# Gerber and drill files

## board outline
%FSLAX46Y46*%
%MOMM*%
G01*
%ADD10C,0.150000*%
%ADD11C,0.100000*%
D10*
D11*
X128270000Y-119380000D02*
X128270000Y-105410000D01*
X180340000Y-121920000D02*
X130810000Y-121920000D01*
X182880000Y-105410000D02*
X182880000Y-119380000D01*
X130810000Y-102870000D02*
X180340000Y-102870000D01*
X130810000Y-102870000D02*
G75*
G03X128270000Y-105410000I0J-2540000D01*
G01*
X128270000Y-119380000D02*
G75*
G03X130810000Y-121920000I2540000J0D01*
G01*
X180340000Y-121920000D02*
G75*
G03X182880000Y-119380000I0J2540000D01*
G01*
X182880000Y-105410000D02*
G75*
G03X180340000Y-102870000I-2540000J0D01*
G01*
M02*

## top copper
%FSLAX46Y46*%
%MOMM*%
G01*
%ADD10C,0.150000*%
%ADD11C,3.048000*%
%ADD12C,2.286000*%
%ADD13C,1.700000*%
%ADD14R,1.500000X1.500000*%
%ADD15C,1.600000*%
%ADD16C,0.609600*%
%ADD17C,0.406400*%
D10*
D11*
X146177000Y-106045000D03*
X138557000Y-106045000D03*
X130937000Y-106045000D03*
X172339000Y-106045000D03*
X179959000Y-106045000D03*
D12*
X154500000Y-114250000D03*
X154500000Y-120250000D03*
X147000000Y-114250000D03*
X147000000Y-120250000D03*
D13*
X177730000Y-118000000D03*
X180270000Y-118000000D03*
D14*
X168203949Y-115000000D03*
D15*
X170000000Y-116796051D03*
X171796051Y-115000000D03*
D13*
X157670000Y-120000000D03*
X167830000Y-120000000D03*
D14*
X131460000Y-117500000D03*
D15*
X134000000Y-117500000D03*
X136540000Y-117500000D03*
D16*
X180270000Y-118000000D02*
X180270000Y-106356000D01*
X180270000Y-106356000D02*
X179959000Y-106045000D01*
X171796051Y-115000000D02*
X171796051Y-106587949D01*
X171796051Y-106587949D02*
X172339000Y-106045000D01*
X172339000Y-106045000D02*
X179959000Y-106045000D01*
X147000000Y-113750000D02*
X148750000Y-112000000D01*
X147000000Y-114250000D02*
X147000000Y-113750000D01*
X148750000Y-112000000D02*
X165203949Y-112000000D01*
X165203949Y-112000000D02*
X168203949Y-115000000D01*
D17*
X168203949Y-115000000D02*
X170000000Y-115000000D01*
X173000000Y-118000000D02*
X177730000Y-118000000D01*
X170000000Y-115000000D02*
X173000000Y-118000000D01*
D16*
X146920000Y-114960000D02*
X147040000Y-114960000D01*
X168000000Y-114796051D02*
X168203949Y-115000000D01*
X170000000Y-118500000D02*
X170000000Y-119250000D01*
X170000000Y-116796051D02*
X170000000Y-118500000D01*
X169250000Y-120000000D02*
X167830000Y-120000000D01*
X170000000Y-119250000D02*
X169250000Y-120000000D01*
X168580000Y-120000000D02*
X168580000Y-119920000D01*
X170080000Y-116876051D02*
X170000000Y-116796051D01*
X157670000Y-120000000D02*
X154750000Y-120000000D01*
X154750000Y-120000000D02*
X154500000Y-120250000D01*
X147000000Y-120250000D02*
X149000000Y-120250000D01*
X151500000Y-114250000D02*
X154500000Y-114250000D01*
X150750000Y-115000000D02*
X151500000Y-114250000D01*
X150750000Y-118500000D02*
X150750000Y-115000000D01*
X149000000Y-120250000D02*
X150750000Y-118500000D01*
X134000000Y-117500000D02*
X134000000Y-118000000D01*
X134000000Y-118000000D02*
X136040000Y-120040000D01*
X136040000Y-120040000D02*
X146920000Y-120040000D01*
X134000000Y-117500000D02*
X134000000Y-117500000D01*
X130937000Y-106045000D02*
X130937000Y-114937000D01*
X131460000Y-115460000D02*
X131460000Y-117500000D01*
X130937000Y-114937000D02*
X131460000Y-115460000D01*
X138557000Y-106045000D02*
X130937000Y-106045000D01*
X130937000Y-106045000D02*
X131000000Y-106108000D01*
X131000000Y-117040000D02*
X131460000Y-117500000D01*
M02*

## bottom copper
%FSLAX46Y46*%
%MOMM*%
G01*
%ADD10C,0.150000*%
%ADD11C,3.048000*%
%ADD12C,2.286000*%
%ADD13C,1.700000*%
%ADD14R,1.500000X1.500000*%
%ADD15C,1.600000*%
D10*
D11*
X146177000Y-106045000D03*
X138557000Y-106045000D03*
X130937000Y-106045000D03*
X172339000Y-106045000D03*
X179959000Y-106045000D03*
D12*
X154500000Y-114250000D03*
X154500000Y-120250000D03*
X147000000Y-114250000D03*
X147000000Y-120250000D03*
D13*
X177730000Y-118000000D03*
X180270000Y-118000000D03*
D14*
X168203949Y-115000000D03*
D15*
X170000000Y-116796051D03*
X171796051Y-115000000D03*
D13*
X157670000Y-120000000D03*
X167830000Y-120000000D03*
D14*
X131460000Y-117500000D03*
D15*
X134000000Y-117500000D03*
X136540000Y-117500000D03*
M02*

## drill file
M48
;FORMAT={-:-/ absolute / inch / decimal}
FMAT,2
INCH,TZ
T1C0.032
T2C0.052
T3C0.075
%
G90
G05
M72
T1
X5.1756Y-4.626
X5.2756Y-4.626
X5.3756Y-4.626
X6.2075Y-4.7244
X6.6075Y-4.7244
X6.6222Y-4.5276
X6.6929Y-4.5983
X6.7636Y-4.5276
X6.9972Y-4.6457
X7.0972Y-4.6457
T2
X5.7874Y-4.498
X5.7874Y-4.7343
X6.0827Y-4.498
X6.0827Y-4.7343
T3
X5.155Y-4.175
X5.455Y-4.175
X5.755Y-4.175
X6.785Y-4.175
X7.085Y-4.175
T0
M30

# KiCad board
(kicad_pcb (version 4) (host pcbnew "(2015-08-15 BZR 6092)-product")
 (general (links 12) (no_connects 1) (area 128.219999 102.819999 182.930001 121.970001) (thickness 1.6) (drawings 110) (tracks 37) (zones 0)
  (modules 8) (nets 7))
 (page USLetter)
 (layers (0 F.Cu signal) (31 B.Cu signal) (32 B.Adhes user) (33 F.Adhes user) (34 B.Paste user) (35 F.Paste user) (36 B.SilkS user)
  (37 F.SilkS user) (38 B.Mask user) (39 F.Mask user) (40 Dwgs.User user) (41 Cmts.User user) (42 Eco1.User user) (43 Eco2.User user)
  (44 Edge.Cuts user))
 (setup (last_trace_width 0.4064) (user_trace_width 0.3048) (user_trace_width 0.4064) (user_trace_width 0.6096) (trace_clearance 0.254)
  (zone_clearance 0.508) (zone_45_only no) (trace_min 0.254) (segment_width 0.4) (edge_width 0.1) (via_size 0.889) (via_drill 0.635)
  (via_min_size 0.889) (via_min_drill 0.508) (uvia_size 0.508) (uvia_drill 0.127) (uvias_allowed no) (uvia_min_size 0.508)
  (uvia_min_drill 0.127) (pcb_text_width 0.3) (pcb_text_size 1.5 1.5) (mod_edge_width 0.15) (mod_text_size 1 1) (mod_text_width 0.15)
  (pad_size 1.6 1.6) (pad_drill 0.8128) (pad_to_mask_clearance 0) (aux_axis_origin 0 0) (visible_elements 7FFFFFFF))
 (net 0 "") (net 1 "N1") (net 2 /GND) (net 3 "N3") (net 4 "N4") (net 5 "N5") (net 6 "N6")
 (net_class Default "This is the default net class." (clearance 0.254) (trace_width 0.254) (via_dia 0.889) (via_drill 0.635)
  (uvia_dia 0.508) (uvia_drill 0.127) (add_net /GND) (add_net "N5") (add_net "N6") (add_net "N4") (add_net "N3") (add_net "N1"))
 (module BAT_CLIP (layer F.Cu) (at 155.575 106.045)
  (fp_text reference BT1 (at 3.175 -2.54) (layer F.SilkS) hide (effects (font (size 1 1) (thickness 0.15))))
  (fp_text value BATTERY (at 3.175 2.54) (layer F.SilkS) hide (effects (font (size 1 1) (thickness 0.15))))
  (pad 1 thru_hole circle (at -9.398 0) (size 3.048 3.048) (drill 1.905) (layers *.Cu *.Mask) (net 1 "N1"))
  (pad 1 thru_hole circle (at -17.018 0) (size 3.048 3.048) (drill 1.905) (layers *.Cu *.Mask) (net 1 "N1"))
  (pad 1 thru_hole circle (at -24.638 0) (size 3.048 3.048) (drill 1.905) (layers *.Cu *.Mask) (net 1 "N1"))
  (pad 2 thru_hole circle (at 16.764 0) (size 3.048 3.048) (drill 1.905) (layers *.Cu *.Mask) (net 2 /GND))
  (pad 2 thru_hole circle (at 24.384 0) (size 3.048 3.048) (drill 1.905) (layers *.Cu *.Mask) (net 2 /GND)))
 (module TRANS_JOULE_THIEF (layer F.Cu) (at 152 117.25 270)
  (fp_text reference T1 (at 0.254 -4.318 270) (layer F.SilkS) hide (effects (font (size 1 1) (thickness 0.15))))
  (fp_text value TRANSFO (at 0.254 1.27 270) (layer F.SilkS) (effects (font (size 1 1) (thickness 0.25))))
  (pad 1 thru_hole circle (at -3 -2.5 270) (size 2.286 2.286) (drill 1.3208) (layers *.Cu B.Mask) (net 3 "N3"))
  (pad 2 thru_hole circle (at 3 -2.5 270) (size 2.286 2.286) (drill 1.3208) (layers *.Cu B.Mask) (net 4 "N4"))
  (pad 3 thru_hole circle (at -3 5 270) (size 2.286 2.286) (drill 1.3208) (layers *.Cu B.Mask) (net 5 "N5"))
  (pad 4 thru_hole circle (at 3 5 270) (size 2.286 2.286) (drill 1.3208) (layers *.Cu B.Mask) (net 3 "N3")))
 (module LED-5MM (layer F.Cu) (at 179 118)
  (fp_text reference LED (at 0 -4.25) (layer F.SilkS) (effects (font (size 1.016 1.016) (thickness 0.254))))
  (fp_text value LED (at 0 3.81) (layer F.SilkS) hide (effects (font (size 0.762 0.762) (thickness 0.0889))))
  (pad 1 thru_hole circle (at -1.27 0) (size 1.7 1.7) (drill 0.8128) (layers *.Cu B.Mask) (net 5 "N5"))
  (pad 2 thru_hole circle (at 1.27 0) (size 1.7 1.7) (drill 0.8128) (layers *.Cu B.Mask) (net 2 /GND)))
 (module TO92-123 (layer F.Cu) (at 170 115 135)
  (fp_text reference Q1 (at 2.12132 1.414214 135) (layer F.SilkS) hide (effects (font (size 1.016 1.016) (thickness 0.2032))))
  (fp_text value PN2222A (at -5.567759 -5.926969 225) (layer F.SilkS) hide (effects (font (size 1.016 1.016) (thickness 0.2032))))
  (pad 3 thru_hole rect (at 1.27 -1.27 180) (size 1.5 1.5) (drill 0.8128) (layers *.Cu B.Mask) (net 5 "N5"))
  (pad 2 thru_hole circle (at -1.27 -1.27 135) (size 1.6 1.6) (drill 0.8128) (layers *.Cu B.Mask) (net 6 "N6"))
  (pad 1 thru_hole circle (at -1.27 1.27 135) (size 1.6 1.6) (drill 0.8128) (layers *.Cu B.Mask) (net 2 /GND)))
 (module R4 (layer F.Cu) (at 162.75 120) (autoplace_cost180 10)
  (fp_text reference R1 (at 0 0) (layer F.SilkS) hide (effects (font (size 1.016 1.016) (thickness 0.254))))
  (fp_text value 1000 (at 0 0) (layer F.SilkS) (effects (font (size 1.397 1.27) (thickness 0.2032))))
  (pad 1 thru_hole circle (at -5.08 0) (size 1.7 1.7) (drill 0.8128) (layers *.Cu B.Mask) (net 4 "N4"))
  (pad 2 thru_hole circle (at 5.08 0) (size 1.7 1.7) (drill 0.8128) (layers *.Cu B.Mask) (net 6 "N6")))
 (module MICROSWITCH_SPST (layer F.Cu) (at 134 117.5)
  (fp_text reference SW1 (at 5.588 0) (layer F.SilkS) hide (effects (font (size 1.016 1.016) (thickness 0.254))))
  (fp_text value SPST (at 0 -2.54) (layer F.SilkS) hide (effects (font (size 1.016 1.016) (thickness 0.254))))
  (pad 1 thru_hole rect (at -2.54 0) (size 1.5 1.5) (drill 0.8128) (layers *.Cu B.Mask) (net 1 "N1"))
  (pad 2 thru_hole circle (at 0 0) (size 1.6 1.6) (drill 0.8128) (layers *.Cu B.Mask) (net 3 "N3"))
  (pad 3 thru_hole circle (at 2.54 0) (size 1.6 1.6) (drill 0.8128) (layers *.Cu B.Mask)))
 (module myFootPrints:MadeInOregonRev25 (layer F.Cu) (at 134 111.5)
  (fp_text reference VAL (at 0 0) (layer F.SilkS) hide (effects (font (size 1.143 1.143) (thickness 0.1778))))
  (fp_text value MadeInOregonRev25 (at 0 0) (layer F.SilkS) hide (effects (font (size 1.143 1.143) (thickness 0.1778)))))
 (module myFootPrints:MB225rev (layer F.Cu) (at 141 111.5)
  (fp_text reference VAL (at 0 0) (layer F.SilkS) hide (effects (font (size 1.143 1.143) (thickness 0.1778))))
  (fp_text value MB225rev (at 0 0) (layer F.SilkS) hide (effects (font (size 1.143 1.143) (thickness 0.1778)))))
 (gr_line (start 128.27 119.38) (end 128.27 105.41) (angle 90) (layer Edge.Cuts) (width 0.1))
 (gr_line (start 180.34 121.92) (end 130.81 121.92) (angle 90) (layer Edge.Cuts) (width 0.1))
 (gr_line (start 182.88 105.41) (end 182.88 119.38) (angle 90) (layer Edge.Cuts) (width 0.1))
 (gr_line (start 130.81 102.87) (end 180.34 102.87) (angle 90) (layer Edge.Cuts) (width 0.1))
 (gr_arc (start 130.81 105.41) (end 128.27 105.41) (angle 90) (layer Edge.Cuts) (width 0.1))
 (gr_arc (start 130.81 119.38) (end 130.81 121.92) (angle 90) (layer Edge.Cuts) (width 0.1))
 (gr_arc (start 180.34 119.38) (end 182.88 119.38) (angle 90) (layer Edge.Cuts) (width 0.1))
 (gr_arc (start 180.34 105.41) (end 180.34 102.87) (angle 90) (layer Edge.Cuts) (width 0.1))
 (segment (start 180.27 118) (end 180.27 106.356) (width 0.6096) (layer F.Cu) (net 2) (status 10))
 (segment (start 180.27 106.356) (end 179.959 106.045) (width 0.6096) (layer F.Cu) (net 2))
 (segment (start 171.796051 115) (end 171.796051 106.587949) (width 0.6096) (layer F.Cu) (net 2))
 (segment (start 171.796051 106.587949) (end 172.339 106.045) (width 0.6096) (layer F.Cu) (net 2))
 (segment (start 172.339 106.045) (end 179.959 106.045) (width 0.6096) (layer F.Cu) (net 2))
 (segment (start 147 113.75) (end 148.75 112) (width 0.6096) (layer F.Cu) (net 5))
 (segment (start 147 114.25) (end 147 113.75) (width 0.6096) (layer F.Cu) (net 5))
 (segment (start 148.75 112) (end 165.203949 112) (width 0.6096) (layer F.Cu) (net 5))
 (segment (start 165.203949 112) (end 168.203949 115) (width 0.6096) (layer F.Cu) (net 5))
 (segment (start 168.203949 115) (end 170 115) (width 0.4064) (layer F.Cu) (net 5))
 (segment (start 173 118) (end 177.73 118) (width 0.4064) (layer F.Cu) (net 5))
 (segment (start 170 115) (end 173 118) (width 0.4064) (layer F.Cu) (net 5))
 (segment (start 146.92 114.96) (end 147.04 114.96) (width 0.6096) (layer F.Cu) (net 5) (status 30))
 (segment (start 168 114.796051) (end 168.203949 115) (width 0.6096) (layer F.Cu) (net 5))
 (segment (start 170 118.5) (end 170 119.25) (width 0.6096) (layer F.Cu) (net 6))
 (segment (start 170 116.796051) (end 170 118.5) (width 0.6096) (layer F.Cu) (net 6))
 (segment (start 169.25 120) (end 167.83 120) (width 0.6096) (layer F.Cu) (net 6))
 (segment (start 170 119.25) (end 169.25 120) (width 0.6096) (layer F.Cu) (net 6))
 (segment (start 168.58 120) (end 168.58 119.92) (width 0.6096) (layer F.Cu) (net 6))
 (segment (start 170.08 116.876051) (end 170 116.796051) (width 0.6096) (layer F.Cu) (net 6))
 (segment (start 157.67 120) (end 154.75 120) (width 0.6096) (layer F.Cu) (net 4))
 (segment (start 154.75 120) (end 154.5 120.25) (width 0.6096) (layer F.Cu) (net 4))
 (segment (start 147 120.25) (end 149 120.25) (width 0.6096) (layer F.Cu) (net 3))
 (segment (start 151.5 114.25) (end 154.5 114.25) (width 0.6096) (layer F.Cu) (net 3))
 (segment (start 150.75 115) (end 151.5 114.25) (width 0.6096) (layer F.Cu) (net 3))
 (segment (start 150.75 118.5) (end 150.75 115) (width 0.6096) (layer F.Cu) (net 3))
 (segment (start 149 120.25) (end 150.75 118.5) (width 0.6096) (layer F.Cu) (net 3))
 (segment (start 134 117.5) (end 134 118) (width 0.6096) (layer F.Cu) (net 3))
 (segment (start 134 118) (end 136.04 120.04) (width 0.6096) (layer F.Cu) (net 3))
 (segment (start 136.04 120.04) (end 146.92 120.04) (width 0.6096) (layer F.Cu) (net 3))
 (segment (start 134 117.5) (end 134 117.5) (width 0.6096) (layer F.Cu) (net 3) (status 10))
 (segment (start 130.937 106.045) (end 130.937 114.937) (width 0.6096) (layer F.Cu) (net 1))
 (segment (start 131.46 115.46) (end 131.46 117.5) (width 0.6096) (layer F.Cu) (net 1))
 (segment (start 130.937 114.937) (end 131.46 115.46) (width 0.6096) (layer F.Cu) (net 1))
 (segment (start 138.557 106.045) (end 130.937 106.045) (width 0.6096) (layer F.Cu) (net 1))
 (segment (start 130.937 106.045) (end 131 106.108) (width 0.6096) (layer F.Cu) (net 1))
 (segment (start 131 117.04) (end 131.46 117.5) (width 0.6096) (layer F.Cu) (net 1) (status 30)))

